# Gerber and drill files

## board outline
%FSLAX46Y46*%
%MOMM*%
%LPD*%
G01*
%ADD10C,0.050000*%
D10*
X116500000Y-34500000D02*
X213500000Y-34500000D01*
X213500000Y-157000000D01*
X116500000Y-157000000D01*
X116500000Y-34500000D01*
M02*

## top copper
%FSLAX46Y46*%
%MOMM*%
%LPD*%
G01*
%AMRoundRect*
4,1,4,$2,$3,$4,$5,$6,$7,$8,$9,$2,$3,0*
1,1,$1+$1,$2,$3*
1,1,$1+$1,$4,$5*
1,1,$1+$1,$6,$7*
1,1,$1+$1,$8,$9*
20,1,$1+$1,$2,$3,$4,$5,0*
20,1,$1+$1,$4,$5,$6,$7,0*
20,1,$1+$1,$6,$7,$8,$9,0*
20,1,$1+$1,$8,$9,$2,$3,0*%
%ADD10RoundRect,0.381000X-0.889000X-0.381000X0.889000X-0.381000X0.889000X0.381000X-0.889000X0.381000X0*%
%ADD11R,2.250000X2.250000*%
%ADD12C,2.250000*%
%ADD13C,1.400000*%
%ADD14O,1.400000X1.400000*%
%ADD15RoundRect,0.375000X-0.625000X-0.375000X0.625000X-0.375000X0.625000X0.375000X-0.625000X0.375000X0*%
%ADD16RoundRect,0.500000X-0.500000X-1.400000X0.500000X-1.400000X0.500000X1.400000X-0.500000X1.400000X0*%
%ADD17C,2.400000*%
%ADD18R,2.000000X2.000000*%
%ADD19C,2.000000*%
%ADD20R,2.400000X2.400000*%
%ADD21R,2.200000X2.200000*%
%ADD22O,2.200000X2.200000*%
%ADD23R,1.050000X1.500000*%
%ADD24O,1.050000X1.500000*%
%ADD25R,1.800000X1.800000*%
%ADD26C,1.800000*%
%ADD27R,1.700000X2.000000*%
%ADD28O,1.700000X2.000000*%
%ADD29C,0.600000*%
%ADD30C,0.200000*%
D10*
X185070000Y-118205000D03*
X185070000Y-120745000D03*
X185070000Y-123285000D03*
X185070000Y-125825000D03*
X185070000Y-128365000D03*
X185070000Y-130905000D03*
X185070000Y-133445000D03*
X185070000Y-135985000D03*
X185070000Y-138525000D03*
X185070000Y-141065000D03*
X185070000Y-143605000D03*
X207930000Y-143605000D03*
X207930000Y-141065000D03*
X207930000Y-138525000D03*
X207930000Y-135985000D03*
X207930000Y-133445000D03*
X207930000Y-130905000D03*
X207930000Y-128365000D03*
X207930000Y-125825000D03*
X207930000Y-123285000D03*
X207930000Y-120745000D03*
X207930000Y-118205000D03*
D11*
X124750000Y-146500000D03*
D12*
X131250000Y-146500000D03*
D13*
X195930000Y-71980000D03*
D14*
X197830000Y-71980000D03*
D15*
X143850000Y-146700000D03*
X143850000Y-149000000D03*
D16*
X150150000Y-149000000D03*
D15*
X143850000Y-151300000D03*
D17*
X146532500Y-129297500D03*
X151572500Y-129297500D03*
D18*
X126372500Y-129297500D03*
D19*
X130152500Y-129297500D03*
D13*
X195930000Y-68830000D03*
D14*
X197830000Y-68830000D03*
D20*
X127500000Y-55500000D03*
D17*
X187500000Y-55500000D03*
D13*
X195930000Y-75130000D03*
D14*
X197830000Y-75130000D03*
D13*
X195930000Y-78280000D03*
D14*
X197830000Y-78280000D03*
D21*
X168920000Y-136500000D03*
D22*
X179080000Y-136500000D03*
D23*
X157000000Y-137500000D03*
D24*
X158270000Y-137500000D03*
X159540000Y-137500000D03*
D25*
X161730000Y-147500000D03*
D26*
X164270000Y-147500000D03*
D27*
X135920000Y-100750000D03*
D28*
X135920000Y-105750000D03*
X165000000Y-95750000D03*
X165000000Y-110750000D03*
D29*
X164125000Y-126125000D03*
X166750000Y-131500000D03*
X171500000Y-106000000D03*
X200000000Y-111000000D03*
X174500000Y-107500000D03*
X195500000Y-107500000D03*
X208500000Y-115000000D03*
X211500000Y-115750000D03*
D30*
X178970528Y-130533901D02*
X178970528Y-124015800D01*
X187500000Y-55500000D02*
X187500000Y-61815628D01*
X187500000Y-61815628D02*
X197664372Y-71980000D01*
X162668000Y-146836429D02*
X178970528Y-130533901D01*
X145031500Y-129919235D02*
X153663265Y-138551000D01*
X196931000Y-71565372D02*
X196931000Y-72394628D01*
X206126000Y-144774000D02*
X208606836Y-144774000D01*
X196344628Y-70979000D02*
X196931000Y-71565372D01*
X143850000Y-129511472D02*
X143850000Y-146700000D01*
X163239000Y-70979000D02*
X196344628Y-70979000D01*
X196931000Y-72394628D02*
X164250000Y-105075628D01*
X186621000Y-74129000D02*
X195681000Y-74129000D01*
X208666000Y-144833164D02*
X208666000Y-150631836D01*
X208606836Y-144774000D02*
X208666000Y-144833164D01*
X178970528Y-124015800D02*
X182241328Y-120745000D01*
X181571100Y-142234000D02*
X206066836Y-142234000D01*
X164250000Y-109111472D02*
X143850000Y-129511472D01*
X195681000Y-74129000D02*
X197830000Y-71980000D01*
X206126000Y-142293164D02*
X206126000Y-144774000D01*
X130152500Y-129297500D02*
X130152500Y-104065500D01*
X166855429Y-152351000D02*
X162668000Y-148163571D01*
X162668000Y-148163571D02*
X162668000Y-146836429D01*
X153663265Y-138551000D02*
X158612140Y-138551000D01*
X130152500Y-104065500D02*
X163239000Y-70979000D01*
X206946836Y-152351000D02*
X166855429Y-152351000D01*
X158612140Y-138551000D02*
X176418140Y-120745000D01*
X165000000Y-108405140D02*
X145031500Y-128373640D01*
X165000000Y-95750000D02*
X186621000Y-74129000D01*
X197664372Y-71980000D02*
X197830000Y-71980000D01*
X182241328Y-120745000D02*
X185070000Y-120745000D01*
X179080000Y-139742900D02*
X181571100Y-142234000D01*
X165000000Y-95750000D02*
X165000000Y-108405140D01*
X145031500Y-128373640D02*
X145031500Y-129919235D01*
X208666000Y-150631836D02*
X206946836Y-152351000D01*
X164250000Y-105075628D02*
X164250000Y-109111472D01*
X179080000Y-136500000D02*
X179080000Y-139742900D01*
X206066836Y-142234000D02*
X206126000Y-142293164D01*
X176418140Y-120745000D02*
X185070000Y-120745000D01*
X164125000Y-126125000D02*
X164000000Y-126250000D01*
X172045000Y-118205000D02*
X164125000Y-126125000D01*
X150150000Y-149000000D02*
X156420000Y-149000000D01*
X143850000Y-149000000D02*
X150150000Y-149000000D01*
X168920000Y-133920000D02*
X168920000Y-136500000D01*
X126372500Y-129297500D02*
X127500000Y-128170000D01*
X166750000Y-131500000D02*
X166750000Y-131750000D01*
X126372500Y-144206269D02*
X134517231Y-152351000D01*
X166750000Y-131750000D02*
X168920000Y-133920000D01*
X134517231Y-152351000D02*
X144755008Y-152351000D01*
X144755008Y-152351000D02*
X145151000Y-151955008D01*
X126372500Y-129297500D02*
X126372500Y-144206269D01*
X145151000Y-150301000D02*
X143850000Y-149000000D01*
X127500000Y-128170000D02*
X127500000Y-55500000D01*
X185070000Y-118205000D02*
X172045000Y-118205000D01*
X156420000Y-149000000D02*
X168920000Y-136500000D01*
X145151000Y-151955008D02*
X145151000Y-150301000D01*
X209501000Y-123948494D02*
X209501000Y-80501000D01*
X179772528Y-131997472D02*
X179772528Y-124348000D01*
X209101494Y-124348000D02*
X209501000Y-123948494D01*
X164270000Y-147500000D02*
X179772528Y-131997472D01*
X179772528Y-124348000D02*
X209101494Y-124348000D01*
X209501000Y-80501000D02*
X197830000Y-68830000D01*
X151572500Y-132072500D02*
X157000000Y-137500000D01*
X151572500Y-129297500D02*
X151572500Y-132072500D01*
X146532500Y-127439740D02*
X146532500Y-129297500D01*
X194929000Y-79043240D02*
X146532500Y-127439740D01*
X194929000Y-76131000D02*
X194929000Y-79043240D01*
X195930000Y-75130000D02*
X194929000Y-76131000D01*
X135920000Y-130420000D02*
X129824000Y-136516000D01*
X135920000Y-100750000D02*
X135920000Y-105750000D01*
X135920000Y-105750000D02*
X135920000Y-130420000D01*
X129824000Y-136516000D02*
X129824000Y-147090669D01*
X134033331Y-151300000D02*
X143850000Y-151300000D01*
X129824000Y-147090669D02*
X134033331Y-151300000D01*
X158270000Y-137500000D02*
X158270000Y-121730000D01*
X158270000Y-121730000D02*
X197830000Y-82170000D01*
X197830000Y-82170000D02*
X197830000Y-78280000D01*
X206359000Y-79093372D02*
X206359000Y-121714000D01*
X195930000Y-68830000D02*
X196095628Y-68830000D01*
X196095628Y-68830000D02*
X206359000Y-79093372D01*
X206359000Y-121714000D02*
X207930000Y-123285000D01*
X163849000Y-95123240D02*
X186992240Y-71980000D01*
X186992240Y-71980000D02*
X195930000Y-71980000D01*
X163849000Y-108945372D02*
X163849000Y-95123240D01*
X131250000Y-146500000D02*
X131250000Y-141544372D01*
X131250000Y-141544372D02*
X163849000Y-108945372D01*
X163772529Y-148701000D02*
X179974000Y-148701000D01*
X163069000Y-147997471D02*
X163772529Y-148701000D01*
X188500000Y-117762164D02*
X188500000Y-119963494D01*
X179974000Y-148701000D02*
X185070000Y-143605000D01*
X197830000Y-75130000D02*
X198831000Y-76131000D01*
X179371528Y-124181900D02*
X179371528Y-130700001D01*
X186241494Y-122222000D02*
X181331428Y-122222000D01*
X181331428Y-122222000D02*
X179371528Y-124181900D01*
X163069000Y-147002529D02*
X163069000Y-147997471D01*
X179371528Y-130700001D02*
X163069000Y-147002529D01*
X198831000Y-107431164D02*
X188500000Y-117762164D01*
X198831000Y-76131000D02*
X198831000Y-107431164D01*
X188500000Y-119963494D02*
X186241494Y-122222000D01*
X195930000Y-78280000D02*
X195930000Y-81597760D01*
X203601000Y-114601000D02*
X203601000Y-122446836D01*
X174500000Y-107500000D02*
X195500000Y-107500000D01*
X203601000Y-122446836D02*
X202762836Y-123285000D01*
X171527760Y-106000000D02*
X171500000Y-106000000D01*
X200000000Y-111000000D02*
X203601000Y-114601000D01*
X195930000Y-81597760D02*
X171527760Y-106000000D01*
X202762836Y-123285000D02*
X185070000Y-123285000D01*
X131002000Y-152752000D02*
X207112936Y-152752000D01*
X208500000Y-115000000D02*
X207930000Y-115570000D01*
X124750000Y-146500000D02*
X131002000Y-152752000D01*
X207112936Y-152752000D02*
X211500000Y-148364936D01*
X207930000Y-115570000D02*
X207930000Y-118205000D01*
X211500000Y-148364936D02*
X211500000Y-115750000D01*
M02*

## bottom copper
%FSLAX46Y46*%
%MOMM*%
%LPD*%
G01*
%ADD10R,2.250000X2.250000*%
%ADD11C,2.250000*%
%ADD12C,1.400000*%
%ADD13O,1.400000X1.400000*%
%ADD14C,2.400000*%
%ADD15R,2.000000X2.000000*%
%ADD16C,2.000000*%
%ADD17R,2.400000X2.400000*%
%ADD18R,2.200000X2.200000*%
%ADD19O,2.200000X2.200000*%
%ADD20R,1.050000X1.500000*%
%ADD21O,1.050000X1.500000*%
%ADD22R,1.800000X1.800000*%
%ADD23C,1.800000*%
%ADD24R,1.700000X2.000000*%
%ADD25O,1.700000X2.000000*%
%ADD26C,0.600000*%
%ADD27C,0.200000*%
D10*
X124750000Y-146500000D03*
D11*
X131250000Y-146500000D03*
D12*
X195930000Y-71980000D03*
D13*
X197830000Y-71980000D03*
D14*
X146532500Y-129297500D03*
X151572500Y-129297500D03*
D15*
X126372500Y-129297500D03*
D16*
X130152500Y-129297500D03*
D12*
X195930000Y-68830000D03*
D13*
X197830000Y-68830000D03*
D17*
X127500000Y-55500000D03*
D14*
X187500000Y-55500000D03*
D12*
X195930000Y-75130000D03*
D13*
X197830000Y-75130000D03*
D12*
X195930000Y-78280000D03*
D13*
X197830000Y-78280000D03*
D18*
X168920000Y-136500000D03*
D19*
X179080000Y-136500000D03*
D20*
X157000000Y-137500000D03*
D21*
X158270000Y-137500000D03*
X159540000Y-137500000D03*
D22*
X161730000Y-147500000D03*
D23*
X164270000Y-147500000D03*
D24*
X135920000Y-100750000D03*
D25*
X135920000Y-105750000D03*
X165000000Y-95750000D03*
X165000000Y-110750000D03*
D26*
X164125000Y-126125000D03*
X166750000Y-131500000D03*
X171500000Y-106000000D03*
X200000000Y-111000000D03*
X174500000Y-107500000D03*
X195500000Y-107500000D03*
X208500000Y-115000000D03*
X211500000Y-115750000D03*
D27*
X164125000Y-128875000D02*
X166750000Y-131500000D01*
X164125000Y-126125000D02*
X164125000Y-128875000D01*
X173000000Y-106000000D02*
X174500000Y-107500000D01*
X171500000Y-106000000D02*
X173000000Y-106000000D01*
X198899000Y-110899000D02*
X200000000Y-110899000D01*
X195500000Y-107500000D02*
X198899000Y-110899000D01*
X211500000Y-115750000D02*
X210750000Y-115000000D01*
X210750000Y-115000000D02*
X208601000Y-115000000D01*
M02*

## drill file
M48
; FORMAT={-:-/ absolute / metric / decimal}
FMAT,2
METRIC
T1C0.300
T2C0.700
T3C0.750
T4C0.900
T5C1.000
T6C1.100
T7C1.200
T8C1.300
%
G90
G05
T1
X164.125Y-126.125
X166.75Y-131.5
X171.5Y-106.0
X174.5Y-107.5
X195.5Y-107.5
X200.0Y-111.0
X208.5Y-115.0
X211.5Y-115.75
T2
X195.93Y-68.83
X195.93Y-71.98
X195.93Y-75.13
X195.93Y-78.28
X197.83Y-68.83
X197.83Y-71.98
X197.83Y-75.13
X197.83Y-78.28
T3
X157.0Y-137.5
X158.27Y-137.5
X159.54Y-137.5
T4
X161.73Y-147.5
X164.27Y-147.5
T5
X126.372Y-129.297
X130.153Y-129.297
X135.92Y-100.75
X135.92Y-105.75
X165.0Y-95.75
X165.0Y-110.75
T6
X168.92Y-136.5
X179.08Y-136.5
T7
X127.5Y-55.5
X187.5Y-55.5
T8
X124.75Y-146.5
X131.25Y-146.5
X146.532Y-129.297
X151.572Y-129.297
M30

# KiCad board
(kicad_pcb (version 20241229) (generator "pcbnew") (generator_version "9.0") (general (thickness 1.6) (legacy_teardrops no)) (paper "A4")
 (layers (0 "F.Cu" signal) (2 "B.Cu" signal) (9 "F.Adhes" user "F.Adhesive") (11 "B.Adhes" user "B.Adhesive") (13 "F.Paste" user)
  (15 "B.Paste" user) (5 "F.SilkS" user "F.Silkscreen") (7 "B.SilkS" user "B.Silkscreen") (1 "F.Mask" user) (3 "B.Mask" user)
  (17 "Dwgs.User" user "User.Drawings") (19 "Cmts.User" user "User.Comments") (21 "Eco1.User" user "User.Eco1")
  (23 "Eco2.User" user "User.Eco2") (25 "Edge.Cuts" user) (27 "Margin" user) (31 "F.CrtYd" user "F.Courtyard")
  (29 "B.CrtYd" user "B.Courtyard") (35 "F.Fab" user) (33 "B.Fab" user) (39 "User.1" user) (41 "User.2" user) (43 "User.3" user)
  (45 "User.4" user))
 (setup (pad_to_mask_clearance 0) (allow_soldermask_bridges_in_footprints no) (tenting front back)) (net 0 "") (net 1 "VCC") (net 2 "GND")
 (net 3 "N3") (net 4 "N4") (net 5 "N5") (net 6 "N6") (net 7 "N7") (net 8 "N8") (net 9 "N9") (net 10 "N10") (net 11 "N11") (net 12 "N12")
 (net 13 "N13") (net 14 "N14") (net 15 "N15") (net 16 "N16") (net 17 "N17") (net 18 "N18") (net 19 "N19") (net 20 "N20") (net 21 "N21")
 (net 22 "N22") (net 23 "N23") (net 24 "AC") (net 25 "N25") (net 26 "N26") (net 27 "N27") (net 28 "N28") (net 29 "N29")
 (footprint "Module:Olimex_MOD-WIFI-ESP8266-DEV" (layer "F.Cu") (at 196.5 130.905)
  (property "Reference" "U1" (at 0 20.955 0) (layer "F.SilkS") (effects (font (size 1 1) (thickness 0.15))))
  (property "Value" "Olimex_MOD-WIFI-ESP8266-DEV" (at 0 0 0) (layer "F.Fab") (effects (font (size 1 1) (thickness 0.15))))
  (pad "1" smd roundrect (at -11.43 -12.7) (size 2.54 1.524) (layers "F.Cu" "F.Mask" "F.Paste") (roundrect_rratio 0.25) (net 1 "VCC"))
  (pad "2" smd roundrect (at -11.43 -10.16) (size 2.54 1.524) (layers "F.Cu" "F.Mask" "F.Paste") (roundrect_rratio 0.25) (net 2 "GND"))
  (pad "3" smd roundrect (at -11.43 -7.62) (size 2.54 1.524) (layers "F.Cu" "F.Mask" "F.Paste") (roundrect_rratio 0.25) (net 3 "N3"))
  (pad "4" smd roundrect (at -11.43 -5.08) (size 2.54 1.524) (layers "F.Cu" "F.Mask" "F.Paste") (roundrect_rratio 0.25) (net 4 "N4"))
  (pad "5" smd roundrect (at -11.43 -2.54) (size 2.54 1.524) (layers "F.Cu" "F.Mask" "F.Paste") (roundrect_rratio 0.25) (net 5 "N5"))
  (pad "6" smd roundrect (at -11.43 0) (size 2.54 1.524) (layers "F.Cu" "F.Mask" "F.Paste") (roundrect_rratio 0.25) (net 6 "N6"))
  (pad "7" smd roundrect (at -11.43 2.54) (size 2.54 1.524) (layers "F.Cu" "F.Mask" "F.Paste") (roundrect_rratio 0.25) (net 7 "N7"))
  (pad "8" smd roundrect (at -11.43 5.08) (size 2.54 1.524) (layers "F.Cu" "F.Mask" "F.Paste") (roundrect_rratio 0.25) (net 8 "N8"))
  (pad "9" smd roundrect (at -11.43 7.62) (size 2.54 1.524) (layers "F.Cu" "F.Mask" "F.Paste") (roundrect_rratio 0.25) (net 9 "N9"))
  (pad "10" smd roundrect (at -11.43 10.16) (size 2.54 1.524) (layers "F.Cu" "F.Mask" "F.Paste") (roundrect_rratio 0.25) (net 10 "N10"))
  (pad "11" smd roundrect (at -11.43 12.7) (size 2.54 1.524) (layers "F.Cu" "F.Mask" "F.Paste") (roundrect_rratio 0.25) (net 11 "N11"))
  (pad "12" smd roundrect (at 11.43 12.7) (size 2.54 1.524) (layers "F.Cu" "F.Mask" "F.Paste") (roundrect_rratio 0.25) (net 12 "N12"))
  (pad "13" smd roundrect (at 11.43 10.16) (size 2.54 1.524) (layers "F.Cu" "F.Mask" "F.Paste") (roundrect_rratio 0.25) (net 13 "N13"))
  (pad "14" smd roundrect (at 11.43 7.62) (size 2.54 1.524) (layers "F.Cu" "F.Mask" "F.Paste") (roundrect_rratio 0.25) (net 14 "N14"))
  (pad "15" smd roundrect (at 11.43 5.08) (size 2.54 1.524) (layers "F.Cu" "F.Mask" "F.Paste") (roundrect_rratio 0.25) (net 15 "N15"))
  (pad "16" smd roundrect (at 11.43 2.54) (size 2.54 1.524) (layers "F.Cu" "F.Mask" "F.Paste") (roundrect_rratio 0.25) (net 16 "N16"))
  (pad "17" smd roundrect (at 11.43 0) (size 2.54 1.524) (layers "F.Cu" "F.Mask" "F.Paste") (roundrect_rratio 0.25) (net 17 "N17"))
  (pad "18" smd roundrect (at 11.43 -2.54) (size 2.54 1.524) (layers "F.Cu" "F.Mask" "F.Paste") (roundrect_rratio 0.25) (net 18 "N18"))
  (pad "19" smd roundrect (at 11.43 -5.08) (size 2.54 1.524) (layers "F.Cu" "F.Mask" "F.Paste") (roundrect_rratio 0.25) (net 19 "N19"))
  (pad "20" smd roundrect (at 11.43 -7.62) (size 2.54 1.524) (layers "F.Cu" "F.Mask" "F.Paste") (roundrect_rratio 0.25) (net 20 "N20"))
  (pad "21" smd roundrect (at 11.43 -10.16) (size 2.54 1.524) (layers "F.Cu" "F.Mask" "F.Paste") (roundrect_rratio 0.25) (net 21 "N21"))
  (pad "22" smd roundrect (at 11.43 -12.7) (size 2.54 1.524) (layers "F.Cu" "F.Mask" "F.Paste") (roundrect_rratio 0.25) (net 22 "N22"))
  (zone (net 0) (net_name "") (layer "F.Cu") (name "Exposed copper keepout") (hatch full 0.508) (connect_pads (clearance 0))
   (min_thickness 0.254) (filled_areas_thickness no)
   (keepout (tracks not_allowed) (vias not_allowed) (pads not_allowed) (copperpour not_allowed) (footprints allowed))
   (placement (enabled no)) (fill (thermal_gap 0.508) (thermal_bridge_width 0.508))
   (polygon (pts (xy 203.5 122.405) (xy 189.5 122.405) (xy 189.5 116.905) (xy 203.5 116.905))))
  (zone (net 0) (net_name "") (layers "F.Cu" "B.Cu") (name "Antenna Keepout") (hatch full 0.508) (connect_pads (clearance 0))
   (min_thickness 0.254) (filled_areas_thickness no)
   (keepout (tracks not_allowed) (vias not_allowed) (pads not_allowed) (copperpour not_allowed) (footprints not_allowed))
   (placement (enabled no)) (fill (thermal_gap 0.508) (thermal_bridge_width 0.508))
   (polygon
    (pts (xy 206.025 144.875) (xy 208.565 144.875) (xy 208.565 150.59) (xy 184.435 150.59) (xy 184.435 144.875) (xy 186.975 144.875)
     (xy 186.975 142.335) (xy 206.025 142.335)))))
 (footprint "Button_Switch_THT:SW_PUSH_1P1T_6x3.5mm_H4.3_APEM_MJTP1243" (layer "F.Cu") (at 124.75 146.5)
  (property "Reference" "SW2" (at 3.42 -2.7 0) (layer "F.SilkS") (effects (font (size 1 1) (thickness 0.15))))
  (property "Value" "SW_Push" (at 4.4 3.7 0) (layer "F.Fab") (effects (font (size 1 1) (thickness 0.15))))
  (pad "1" thru_hole rect (at 0 0 90) (size 2.25 2.25) (drill 1.3) (layers "*.Cu" "*.Mask") (remove_unused_layers no) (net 22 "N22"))
  (pad "2" thru_hole circle (at 6.5 0 90) (size 2.25 2.25) (drill 1.3) (layers "*.Cu" "*.Mask") (remove_unused_layers no) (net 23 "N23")))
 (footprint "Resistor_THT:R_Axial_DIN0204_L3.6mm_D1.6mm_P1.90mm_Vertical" (layer "F.Cu") (at 195.93 71.98)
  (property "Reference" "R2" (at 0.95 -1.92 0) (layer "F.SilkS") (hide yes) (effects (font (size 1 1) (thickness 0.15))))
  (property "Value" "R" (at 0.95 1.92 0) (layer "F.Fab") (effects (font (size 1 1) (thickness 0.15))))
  (pad "1" thru_hole circle (at 0 0) (size 1.4 1.4) (drill 0.7) (layers "*.Cu" "*.Mask") (remove_unused_layers no) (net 23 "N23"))
  (pad "2" thru_hole oval (at 1.9 0) (size 1.4 1.4) (drill 0.7) (layers "*.Cu" "*.Mask") (remove_unused_layers no) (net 2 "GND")))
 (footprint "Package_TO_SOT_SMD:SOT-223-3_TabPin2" (layer "F.Cu") (at 147 149)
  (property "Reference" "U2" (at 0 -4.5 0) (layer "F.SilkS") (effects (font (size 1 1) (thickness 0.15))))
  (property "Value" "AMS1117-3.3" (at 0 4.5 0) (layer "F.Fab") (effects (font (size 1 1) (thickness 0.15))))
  (pad "1" smd roundrect (at -3.15 -2.3) (size 2 1.5) (layers "F.Cu" "F.Mask" "F.Paste") (roundrect_rratio 0.25) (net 2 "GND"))
  (pad "2" smd roundrect (at -3.15 0) (size 2 1.5) (layers "F.Cu" "F.Mask" "F.Paste") (roundrect_rratio 0.25) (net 1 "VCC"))
  (pad "2" smd roundrect (at 3.15 0) (size 2 3.8) (layers "F.Cu" "F.Mask" "F.Paste") (roundrect_rratio 0.25) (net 1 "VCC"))
  (pad "3" smd roundrect (at -3.15 2.3) (size 2 1.5) (layers "F.Cu" "F.Mask" "F.Paste") (roundrect_rratio 0.25) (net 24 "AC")))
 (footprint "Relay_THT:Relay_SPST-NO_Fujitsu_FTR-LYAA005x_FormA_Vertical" (layer "F.Cu") (at 126.3725 129.2975)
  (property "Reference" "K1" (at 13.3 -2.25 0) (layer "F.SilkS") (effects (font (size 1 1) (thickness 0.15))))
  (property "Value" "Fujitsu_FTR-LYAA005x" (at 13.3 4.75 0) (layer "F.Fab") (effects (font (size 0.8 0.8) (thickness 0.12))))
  (pad "13" thru_hole circle (at 20.16 0) (size 2.4 2.4) (drill 1.3) (layers "*.Cu" "*.Mask") (remove_unused_layers no) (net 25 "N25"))
  (pad "14" thru_hole circle (at 25.2 0) (size 2.4 2.4) (drill 1.3) (layers "*.Cu" "*.Mask") (remove_unused_layers no) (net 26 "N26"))
  (pad "A1" thru_hole rect (at 0 0) (size 2 2) (drill 1) (layers "*.Cu" "*.Mask") (remove_unused_layers no) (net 1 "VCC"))
  (pad "A2" thru_hole circle (at 3.78 0) (size 2 2) (drill 1) (layers "*.Cu" "*.Mask") (remove_unused_layers no) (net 2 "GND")))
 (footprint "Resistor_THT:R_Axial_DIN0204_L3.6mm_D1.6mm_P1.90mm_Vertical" (layer "F.Cu") (at 195.93 68.83)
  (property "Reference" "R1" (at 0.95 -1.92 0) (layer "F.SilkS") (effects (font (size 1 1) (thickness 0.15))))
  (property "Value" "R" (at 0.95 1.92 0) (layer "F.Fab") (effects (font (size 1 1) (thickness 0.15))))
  (pad "1" thru_hole circle (at 0 0) (size 1.4 1.4) (drill 0.7) (layers "*.Cu" "*.Mask") (remove_unused_layers no) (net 20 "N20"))
  (pad "2" thru_hole oval (at 1.9 0) (size 1.4 1.4) (drill 0.7) (layers "*.Cu" "*.Mask") (remove_unused_layers no) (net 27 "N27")))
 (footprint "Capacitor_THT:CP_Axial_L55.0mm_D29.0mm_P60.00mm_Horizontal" (layer "F.Cu") (at 127.5 55.5)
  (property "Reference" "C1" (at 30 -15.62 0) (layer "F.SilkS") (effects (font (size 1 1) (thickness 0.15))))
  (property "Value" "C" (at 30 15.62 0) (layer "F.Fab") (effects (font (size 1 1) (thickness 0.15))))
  (pad "1" thru_hole rect (at 0 0) (size 2.4 2.4) (drill 1.2) (layers "*.Cu" "*.Mask") (remove_unused_layers no) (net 1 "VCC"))
  (pad "2" thru_hole circle (at 60 0) (size 2.4 2.4) (drill 1.2) (layers "*.Cu" "*.Mask") (remove_unused_layers no) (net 2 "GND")))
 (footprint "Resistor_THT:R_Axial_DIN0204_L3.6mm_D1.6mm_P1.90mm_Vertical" (layer "F.Cu") (at 195.93 75.13)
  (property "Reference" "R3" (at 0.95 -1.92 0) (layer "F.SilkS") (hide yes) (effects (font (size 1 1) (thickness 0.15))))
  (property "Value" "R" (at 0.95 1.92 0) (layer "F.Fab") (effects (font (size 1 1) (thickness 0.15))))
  (pad "1" thru_hole circle (at 0 0) (size 1.4 1.4) (drill 0.7) (layers "*.Cu" "*.Mask") (remove_unused_layers no) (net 25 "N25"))
  (pad "2" thru_hole oval (at 1.9 0) (size 1.4 1.4) (drill 0.7) (layers "*.Cu" "*.Mask") (remove_unused_layers no) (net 11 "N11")))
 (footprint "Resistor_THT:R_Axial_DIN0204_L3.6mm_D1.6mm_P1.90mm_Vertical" (layer "F.Cu") (at 195.93 78.28)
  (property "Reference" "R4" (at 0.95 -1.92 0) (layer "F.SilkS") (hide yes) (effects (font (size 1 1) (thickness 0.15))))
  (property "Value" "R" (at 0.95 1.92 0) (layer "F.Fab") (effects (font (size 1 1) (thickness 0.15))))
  (pad "1" thru_hole circle (at 0 0) (size 1.4 1.4) (drill 0.7) (layers "*.Cu" "*.Mask") (remove_unused_layers no) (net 3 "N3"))
  (pad "2" thru_hole oval (at 1.9 0) (size 1.4 1.4) (drill 0.7) (layers "*.Cu" "*.Mask") (remove_unused_layers no) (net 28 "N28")))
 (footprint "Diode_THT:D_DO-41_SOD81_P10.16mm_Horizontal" (layer "F.Cu") (at 168.92 136.5)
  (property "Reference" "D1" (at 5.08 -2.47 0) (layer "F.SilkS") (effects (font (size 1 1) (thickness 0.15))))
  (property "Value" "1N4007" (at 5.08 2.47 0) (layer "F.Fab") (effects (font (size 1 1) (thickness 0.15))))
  (pad "1" thru_hole rect (at 0 0) (size 2.2 2.2) (drill 1.1) (layers "*.Cu" "*.Mask") (remove_unused_layers no) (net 1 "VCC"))
  (pad "2" thru_hole oval (at 10.16 0) (size 2.2 2.2) (drill 1.1) (layers "*.Cu" "*.Mask") (remove_unused_layers no) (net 2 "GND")))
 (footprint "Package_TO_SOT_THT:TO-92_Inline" (layer "F.Cu") (at 157 137.5)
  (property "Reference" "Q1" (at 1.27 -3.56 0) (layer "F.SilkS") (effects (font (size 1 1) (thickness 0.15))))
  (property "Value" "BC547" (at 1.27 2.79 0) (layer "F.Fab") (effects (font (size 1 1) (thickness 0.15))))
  (pad "1" thru_hole rect (at 0 0) (size 1.05 1.5) (drill 0.75) (layers "*.Cu" "*.Mask") (remove_unused_layers no) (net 26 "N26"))
  (pad "2" thru_hole oval (at 1.27 0) (size 1.05 1.5) (drill 0.75) (layers "*.Cu" "*.Mask") (remove_unused_layers no) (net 28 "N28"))
  (pad "3" thru_hole oval (at 2.54 0) (size 1.05 1.5) (drill 0.75) (layers "*.Cu" "*.Mask") (remove_unused_layers no) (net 2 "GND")))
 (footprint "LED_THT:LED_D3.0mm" (layer "F.Cu") (at 161.73 147.5)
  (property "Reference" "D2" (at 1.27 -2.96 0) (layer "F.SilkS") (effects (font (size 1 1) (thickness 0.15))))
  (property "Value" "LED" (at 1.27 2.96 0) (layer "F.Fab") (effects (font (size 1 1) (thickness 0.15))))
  (pad "1" thru_hole rect (at 0 0) (size 1.8 1.8) (drill 0.9) (layers "*.Cu" "*.Mask") (remove_unused_layers no) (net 2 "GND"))
  (pad "2" thru_hole circle (at 2.54 0) (size 1.8 1.8) (drill 0.9) (layers "*.Cu" "*.Mask") (remove_unused_layers no) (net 27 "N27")))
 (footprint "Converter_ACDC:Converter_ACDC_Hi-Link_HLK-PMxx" (layer "F.Cu") (at 135.92 100.75)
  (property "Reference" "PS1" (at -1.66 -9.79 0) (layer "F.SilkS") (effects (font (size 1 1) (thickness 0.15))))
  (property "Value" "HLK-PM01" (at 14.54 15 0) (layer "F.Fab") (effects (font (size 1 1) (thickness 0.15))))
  (pad "1" thru_hole rect (at 0 0) (size 1.7 2) (drill 1) (layers "*.Cu" "*.Mask") (remove_unused_layers no) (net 24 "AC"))
  (pad "2" thru_hole oval (at 0 5) (size 1.7 2) (drill 1) (layers "*.Cu" "*.Mask") (remove_unused_layers no) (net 24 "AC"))
  (pad "3" thru_hole oval (at 29.08 -5) (size 1.7 2) (drill 1) (layers "*.Cu" "*.Mask") (remove_unused_layers no) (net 2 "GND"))
  (pad "4" thru_hole oval (at 29.08 10) (size 1.7 2) (drill 1) (layers "*.Cu" "*.Mask") (remove_unused_layers no) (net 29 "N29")))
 (gr_rect (start 116.5 34.5) (end 213.5 157) (stroke (width 0.05) (type default)) (fill no) (layer "Edge.Cuts"))
 (segment (start 178.970528 130.533901) (end 178.970528 124.0158) (width 0.2) (layer "F.Cu") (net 2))
 (segment (start 187.5 55.5) (end 187.5 61.815628) (width 0.2) (layer "F.Cu") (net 2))
 (segment (start 187.5 61.815628) (end 197.664372 71.98) (width 0.2) (layer "F.Cu") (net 2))
 (segment (start 162.668 146.836429) (end 178.970528 130.533901) (width 0.2) (layer "F.Cu") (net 2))
 (segment (start 145.0315 129.919235) (end 153.663265 138.551) (width 0.2) (layer "F.Cu") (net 2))
 (segment (start 196.931 71.565372) (end 196.931 72.394628) (width 0.2) (layer "F.Cu") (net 2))
 (segment (start 206.126 144.774) (end 208.606836 144.774) (width 0.2) (layer "F.Cu") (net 2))
 (segment (start 196.344628 70.979) (end 196.931 71.565372) (width 0.2) (layer "F.Cu") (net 2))
 (segment (start 143.85 129.511472) (end 143.85 146.7) (width 0.2) (layer "F.Cu") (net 2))
 (segment (start 163.239 70.979) (end 196.344628 70.979) (width 0.2) (layer "F.Cu") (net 2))
 (segment (start 196.931 72.394628) (end 164.25 105.075628) (width 0.2) (layer "F.Cu") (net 2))
 (segment (start 186.621 74.129) (end 195.681 74.129) (width 0.2) (layer "F.Cu") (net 2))
 (segment (start 208.666 144.833164) (end 208.666 150.631836) (width 0.2) (layer "F.Cu") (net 2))
 (segment (start 208.606836 144.774) (end 208.666 144.833164) (width 0.2) (layer "F.Cu") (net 2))
 (segment (start 178.970528 124.0158) (end 182.241328 120.745) (width 0.2) (layer "F.Cu") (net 2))
 (segment (start 181.5711 142.234) (end 206.066836 142.234) (width 0.2) (layer "F.Cu") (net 2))
 (segment (start 164.25 109.111472) (end 143.85 129.511472) (width 0.2) (layer "F.Cu") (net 2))
 (segment (start 195.681 74.129) (end 197.83 71.98) (width 0.2) (layer "F.Cu") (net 2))
 (segment (start 206.126 142.293164) (end 206.126 144.774) (width 0.2) (layer "F.Cu") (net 2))
 (segment (start 130.1525 129.2975) (end 130.1525 104.0655) (width 0.2) (layer "F.Cu") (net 2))
 (segment (start 166.855429 152.351) (end 162.668 148.163571) (width 0.2) (layer "F.Cu") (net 2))
 (segment (start 162.668 148.163571) (end 162.668 146.836429) (width 0.2) (layer "F.Cu") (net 2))
 (segment (start 153.663265 138.551) (end 158.61214 138.551) (width 0.2) (layer "F.Cu") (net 2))
 (segment (start 130.1525 104.0655) (end 163.239 70.979) (width 0.2) (layer "F.Cu") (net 2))
 (segment (start 206.946836 152.351) (end 166.855429 152.351) (width 0.2) (layer "F.Cu") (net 2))
 (segment (start 158.61214 138.551) (end 176.41814 120.745) (width 0.2) (layer "F.Cu") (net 2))
 (segment (start 165 108.40514) (end 145.0315 128.37364) (width 0.2) (layer "F.Cu") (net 2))
 (segment (start 165 95.75) (end 186.621 74.129) (width 0.2) (layer "F.Cu") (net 2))
 (segment (start 197.664372 71.98) (end 197.83 71.98) (width 0.2) (layer "F.Cu") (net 2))
 (segment (start 182.241328 120.745) (end 185.07 120.745) (width 0.2) (layer "F.Cu") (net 2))
 (segment (start 179.08 139.7429) (end 181.5711 142.234) (width 0.2) (layer "F.Cu") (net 2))
 (segment (start 165 95.75) (end 165 108.40514) (width 0.2) (layer "F.Cu") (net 2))
 (segment (start 145.0315 128.37364) (end 145.0315 129.919235) (width 0.2) (layer "F.Cu") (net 2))
 (segment (start 208.666 150.631836) (end 206.946836 152.351) (width 0.2) (layer "F.Cu") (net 2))
 (segment (start 164.25 105.075628) (end 164.25 109.111472) (width 0.2) (layer "F.Cu") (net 2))
 (segment (start 179.08 136.5) (end 179.08 139.7429) (width 0.2) (layer "F.Cu") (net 2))
 (segment (start 206.066836 142.234) (end 206.126 142.293164) (width 0.2) (layer "F.Cu") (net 2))
 (segment (start 176.41814 120.745) (end 185.07 120.745) (width 0.2) (layer "F.Cu") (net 2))
 (segment (start 164.125 126.125) (end 164 126.25) (width 0.2) (layer "F.Cu") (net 1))
 (segment (start 172.045 118.205) (end 164.125 126.125) (width 0.2) (layer "F.Cu") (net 1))
 (segment (start 150.15 149) (end 156.42 149) (width 0.2) (layer "F.Cu") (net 1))
 (segment (start 143.85 149) (end 150.15 149) (width 0.2) (layer "F.Cu") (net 1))
 (segment (start 168.92 133.92) (end 168.92 136.5) (width 0.2) (layer "F.Cu") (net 1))
 (segment (start 126.3725 129.2975) (end 127.5 128.17) (width 0.2) (layer "F.Cu") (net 1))
 (segment (start 166.75 131.5) (end 166.75 131.75) (width 0.2) (layer "F.Cu") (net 1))
 (segment (start 126.3725 144.206269) (end 134.517231 152.351) (width 0.2) (layer "F.Cu") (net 1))
 (segment (start 166.75 131.75) (end 168.92 133.92) (width 0.2) (layer "F.Cu") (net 1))
 (segment (start 134.517231 152.351) (end 144.755008 152.351) (width 0.2) (layer "F.Cu") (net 1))
 (segment (start 144.755008 152.351) (end 145.151 151.955008) (width 0.2) (layer "F.Cu") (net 1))
 (segment (start 126.3725 129.2975) (end 126.3725 144.206269) (width 0.2) (layer "F.Cu") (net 1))
 (segment (start 145.151 150.301) (end 143.85 149) (width 0.2) (layer "F.Cu") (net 1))
 (segment (start 127.5 128.17) (end 127.5 55.5) (width 0.2) (layer "F.Cu") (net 1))
 (segment (start 185.07 118.205) (end 172.045 118.205) (width 0.2) (layer "F.Cu") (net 1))
 (segment (start 156.42 149) (end 168.92 136.5) (width 0.2) (layer "F.Cu") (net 1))
 (segment (start 145.151 151.955008) (end 145.151 150.301) (width 0.2) (layer "F.Cu") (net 1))
 (via (at 164.125 126.125) (size 0.6) (drill 0.3) (layers "F.Cu" "B.Cu") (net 1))
 (via (at 166.75 131.5) (size 0.6) (drill 0.3) (layers "F.Cu" "B.Cu") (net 1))
 (segment (start 164.125 128.875) (end 166.75 131.5) (width 0.2) (layer "B.Cu") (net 1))
 (segment (start 164.125 126.125) (end 164.125 128.875) (width 0.2) (layer "B.Cu") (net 1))
 (segment (start 209.501 123.948494) (end 209.501 80.501) (width 0.2) (layer "F.Cu") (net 27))
 (segment (start 179.772528 131.997472) (end 179.772528 124.348) (width 0.2) (layer "F.Cu") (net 27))
 (segment (start 209.101494 124.348) (end 209.501 123.948494) (width 0.2) (layer "F.Cu") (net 27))
 (segment (start 164.27 147.5) (end 179.772528 131.997472) (width 0.2) (layer "F.Cu") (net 27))
 (segment (start 179.772528 124.348) (end 209.101494 124.348) (width 0.2) (layer "F.Cu") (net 27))
 (segment (start 209.501 80.501) (end 197.83 68.83) (width 0.2) (layer "F.Cu") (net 27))
 (segment (start 151.5725 132.0725) (end 157 137.5) (width 0.2) (layer "F.Cu") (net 26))
 (segment (start 151.5725 129.2975) (end 151.5725 132.0725) (width 0.2) (layer "F.Cu") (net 26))
 (segment (start 146.5325 127.43974) (end 146.5325 129.2975) (width 0.2) (layer "F.Cu") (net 25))
 (segment (start 194.929 79.04324) (end 146.5325 127.43974) (width 0.2) (layer "F.Cu") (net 25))
 (segment (start 194.929 76.131) (end 194.929 79.04324) (width 0.2) (layer "F.Cu") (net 25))
 (segment (start 195.93 75.13) (end 194.929 76.131) (width 0.2) (layer "F.Cu") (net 25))
 (segment (start 135.92 130.42) (end 129.824 136.516) (width 0.2) (layer "F.Cu") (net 24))
 (segment (start 135.92 100.75) (end 135.92 105.75) (width 0.2) (layer "F.Cu") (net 24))
 (segment (start 135.92 105.75) (end 135.92 130.42) (width 0.2) (layer "F.Cu") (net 24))
 (segment (start 129.824 136.516) (end 129.824 147.090669) (width 0.2) (layer "F.Cu") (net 24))
 (segment (start 134.033331 151.3) (end 143.85 151.3) (width 0.2) (layer "F.Cu") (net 24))
 (segment (start 129.824 147.090669) (end 134.033331 151.3) (width 0.2) (layer "F.Cu") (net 24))
 (segment (start 158.27 137.5) (end 158.27 121.73) (width 0.2) (layer "F.Cu") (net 28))
 (segment (start 158.27 121.73) (end 197.83 82.17) (width 0.2) (layer "F.Cu") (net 28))
 (segment (start 197.83 82.17) (end 197.83 78.28) (width 0.2) (layer "F.Cu") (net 28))
 (segment (start 206.359 79.093372) (end 206.359 121.714) (width 0.2) (layer "F.Cu") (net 20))
 (segment (start 195.93 68.83) (end 196.095628 68.83) (width 0.2) (layer "F.Cu") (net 20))
 (segment (start 196.095628 68.83) (end 206.359 79.093372) (width 0.2) (layer "F.Cu") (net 20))
 (segment (start 206.359 121.714) (end 207.93 123.285) (width 0.2) (layer "F.Cu") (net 20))
 (segment (start 163.849 95.12324) (end 186.99224 71.98) (width 0.2) (layer "F.Cu") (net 23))
 (segment (start 186.99224 71.98) (end 195.93 71.98) (width 0.2) (layer "F.Cu") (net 23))
 (segment (start 163.849 108.945372) (end 163.849 95.12324) (width 0.2) (layer "F.Cu") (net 23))
 (segment (start 131.25 146.5) (end 131.25 141.544372) (width 0.2) (layer "F.Cu") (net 23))
 (segment (start 131.25 141.544372) (end 163.849 108.945372) (width 0.2) (layer "F.Cu") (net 23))
 (segment (start 163.772529 148.701) (end 179.974 148.701) (width 0.2) (layer "F.Cu") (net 11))
 (segment (start 163.069 147.997471) (end 163.772529 148.701) (width 0.2) (layer "F.Cu") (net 11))
 (segment (start 188.5 117.762164) (end 188.5 119.963494) (width 0.2) (layer "F.Cu") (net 11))
 (segment (start 179.974 148.701) (end 185.07 143.605) (width 0.2) (layer "F.Cu") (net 11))
 (segment (start 197.83 75.13) (end 198.831 76.131) (width 0.2) (layer "F.Cu") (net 11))
 (segment (start 179.371528 124.1819) (end 179.371528 130.700001) (width 0.2) (layer "F.Cu") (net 11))
 (segment (start 186.241494 122.222) (end 181.331428 122.222) (width 0.2) (layer "F.Cu") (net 11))
 (segment (start 181.331428 122.222) (end 179.371528 124.1819) (width 0.2) (layer "F.Cu") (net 11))
 (segment (start 163.069 147.002529) (end 163.069 147.997471) (width 0.2) (layer "F.Cu") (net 11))
 (segment (start 179.371528 130.700001) (end 163.069 147.002529) (width 0.2) (layer "F.Cu") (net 11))
 (segment (start 198.831 107.431164) (end 188.5 117.762164) (width 0.2) (layer "F.Cu") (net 11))
 (segment (start 198.831 76.131) (end 198.831 107.431164) (width 0.2) (layer "F.Cu") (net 11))
 (segment (start 188.5 119.963494) (end 186.241494 122.222) (width 0.2) (layer "F.Cu") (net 11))
 (segment (start 195.93 78.28) (end 195.93 81.59776) (width 0.2) (layer "F.Cu") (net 3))
 (segment (start 203.601 114.601) (end 203.601 122.446836) (width 0.2) (layer "F.Cu") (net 3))
 (segment (start 174.5 107.5) (end 195.5 107.5) (width 0.2) (layer "F.Cu") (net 3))
 (segment (start 203.601 122.446836) (end 202.762836 123.285) (width 0.2) (layer "F.Cu") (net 3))
 (segment (start 171.52776 106) (end 171.5 106) (width 0.2) (layer "F.Cu") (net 3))
 (segment (start 200 111) (end 203.601 114.601) (width 0.2) (layer "F.Cu") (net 3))
 (segment (start 195.93 81.59776) (end 171.52776 106) (width 0.2) (layer "F.Cu") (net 3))
 (segment (start 202.762836 123.285) (end 185.07 123.285) (width 0.2) (layer "F.Cu") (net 3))
 (via (at 171.5 106) (size 0.6) (drill 0.3) (layers "F.Cu" "B.Cu") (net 3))
 (via (at 200 111) (size 0.6) (drill 0.3) (layers "F.Cu" "B.Cu") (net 3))
 (via (at 174.5 107.5) (size 0.6) (drill 0.3) (layers "F.Cu" "B.Cu") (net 3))
 (via (at 195.5 107.5) (size 0.6) (drill 0.3) (layers "F.Cu" "B.Cu") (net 3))
 (segment (start 173 106) (end 174.5 107.5) (width 0.2) (layer "B.Cu") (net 3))
 (segment (start 171.5 106) (end 173 106) (width 0.2) (layer "B.Cu") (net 3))
 (segment (start 198.899 110.899) (end 200 110.899) (width 0.2) (layer "B.Cu") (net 3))
 (segment (start 195.5 107.5) (end 198.899 110.899) (width 0.2) (layer "B.Cu") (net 3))
 (segment (start 131.002 152.752) (end 207.112936 152.752) (width 0.2) (layer "F.Cu") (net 22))
 (segment (start 208.5 115) (end 207.93 115.57) (width 0.2) (layer "F.Cu") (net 22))
 (segment (start 124.75 146.5) (end 131.002 152.752) (width 0.2) (layer "F.Cu") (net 22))
 (segment (start 207.112936 152.752) (end 211.5 148.364936) (width 0.2) (layer "F.Cu") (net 22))
 (segment (start 207.93 115.57) (end 207.93 118.205) (width 0.2) (layer "F.Cu") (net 22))
 (segment (start 211.5 148.364936) (end 211.5 115.75) (width 0.2) (layer "F.Cu") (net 22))
 (via (at 208.5 115) (size 0.6) (drill 0.3) (layers "F.Cu" "B.Cu") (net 22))
 (via (at 211.5 115.75) (size 0.6) (drill 0.3) (layers "F.Cu" "B.Cu") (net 22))
 (segment (start 211.5 115.75) (end 210.75 115) (width 0.2) (layer "B.Cu") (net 22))
 (segment (start 210.75 115) (end 208.601 115) (width 0.2) (layer "B.Cu") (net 22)))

